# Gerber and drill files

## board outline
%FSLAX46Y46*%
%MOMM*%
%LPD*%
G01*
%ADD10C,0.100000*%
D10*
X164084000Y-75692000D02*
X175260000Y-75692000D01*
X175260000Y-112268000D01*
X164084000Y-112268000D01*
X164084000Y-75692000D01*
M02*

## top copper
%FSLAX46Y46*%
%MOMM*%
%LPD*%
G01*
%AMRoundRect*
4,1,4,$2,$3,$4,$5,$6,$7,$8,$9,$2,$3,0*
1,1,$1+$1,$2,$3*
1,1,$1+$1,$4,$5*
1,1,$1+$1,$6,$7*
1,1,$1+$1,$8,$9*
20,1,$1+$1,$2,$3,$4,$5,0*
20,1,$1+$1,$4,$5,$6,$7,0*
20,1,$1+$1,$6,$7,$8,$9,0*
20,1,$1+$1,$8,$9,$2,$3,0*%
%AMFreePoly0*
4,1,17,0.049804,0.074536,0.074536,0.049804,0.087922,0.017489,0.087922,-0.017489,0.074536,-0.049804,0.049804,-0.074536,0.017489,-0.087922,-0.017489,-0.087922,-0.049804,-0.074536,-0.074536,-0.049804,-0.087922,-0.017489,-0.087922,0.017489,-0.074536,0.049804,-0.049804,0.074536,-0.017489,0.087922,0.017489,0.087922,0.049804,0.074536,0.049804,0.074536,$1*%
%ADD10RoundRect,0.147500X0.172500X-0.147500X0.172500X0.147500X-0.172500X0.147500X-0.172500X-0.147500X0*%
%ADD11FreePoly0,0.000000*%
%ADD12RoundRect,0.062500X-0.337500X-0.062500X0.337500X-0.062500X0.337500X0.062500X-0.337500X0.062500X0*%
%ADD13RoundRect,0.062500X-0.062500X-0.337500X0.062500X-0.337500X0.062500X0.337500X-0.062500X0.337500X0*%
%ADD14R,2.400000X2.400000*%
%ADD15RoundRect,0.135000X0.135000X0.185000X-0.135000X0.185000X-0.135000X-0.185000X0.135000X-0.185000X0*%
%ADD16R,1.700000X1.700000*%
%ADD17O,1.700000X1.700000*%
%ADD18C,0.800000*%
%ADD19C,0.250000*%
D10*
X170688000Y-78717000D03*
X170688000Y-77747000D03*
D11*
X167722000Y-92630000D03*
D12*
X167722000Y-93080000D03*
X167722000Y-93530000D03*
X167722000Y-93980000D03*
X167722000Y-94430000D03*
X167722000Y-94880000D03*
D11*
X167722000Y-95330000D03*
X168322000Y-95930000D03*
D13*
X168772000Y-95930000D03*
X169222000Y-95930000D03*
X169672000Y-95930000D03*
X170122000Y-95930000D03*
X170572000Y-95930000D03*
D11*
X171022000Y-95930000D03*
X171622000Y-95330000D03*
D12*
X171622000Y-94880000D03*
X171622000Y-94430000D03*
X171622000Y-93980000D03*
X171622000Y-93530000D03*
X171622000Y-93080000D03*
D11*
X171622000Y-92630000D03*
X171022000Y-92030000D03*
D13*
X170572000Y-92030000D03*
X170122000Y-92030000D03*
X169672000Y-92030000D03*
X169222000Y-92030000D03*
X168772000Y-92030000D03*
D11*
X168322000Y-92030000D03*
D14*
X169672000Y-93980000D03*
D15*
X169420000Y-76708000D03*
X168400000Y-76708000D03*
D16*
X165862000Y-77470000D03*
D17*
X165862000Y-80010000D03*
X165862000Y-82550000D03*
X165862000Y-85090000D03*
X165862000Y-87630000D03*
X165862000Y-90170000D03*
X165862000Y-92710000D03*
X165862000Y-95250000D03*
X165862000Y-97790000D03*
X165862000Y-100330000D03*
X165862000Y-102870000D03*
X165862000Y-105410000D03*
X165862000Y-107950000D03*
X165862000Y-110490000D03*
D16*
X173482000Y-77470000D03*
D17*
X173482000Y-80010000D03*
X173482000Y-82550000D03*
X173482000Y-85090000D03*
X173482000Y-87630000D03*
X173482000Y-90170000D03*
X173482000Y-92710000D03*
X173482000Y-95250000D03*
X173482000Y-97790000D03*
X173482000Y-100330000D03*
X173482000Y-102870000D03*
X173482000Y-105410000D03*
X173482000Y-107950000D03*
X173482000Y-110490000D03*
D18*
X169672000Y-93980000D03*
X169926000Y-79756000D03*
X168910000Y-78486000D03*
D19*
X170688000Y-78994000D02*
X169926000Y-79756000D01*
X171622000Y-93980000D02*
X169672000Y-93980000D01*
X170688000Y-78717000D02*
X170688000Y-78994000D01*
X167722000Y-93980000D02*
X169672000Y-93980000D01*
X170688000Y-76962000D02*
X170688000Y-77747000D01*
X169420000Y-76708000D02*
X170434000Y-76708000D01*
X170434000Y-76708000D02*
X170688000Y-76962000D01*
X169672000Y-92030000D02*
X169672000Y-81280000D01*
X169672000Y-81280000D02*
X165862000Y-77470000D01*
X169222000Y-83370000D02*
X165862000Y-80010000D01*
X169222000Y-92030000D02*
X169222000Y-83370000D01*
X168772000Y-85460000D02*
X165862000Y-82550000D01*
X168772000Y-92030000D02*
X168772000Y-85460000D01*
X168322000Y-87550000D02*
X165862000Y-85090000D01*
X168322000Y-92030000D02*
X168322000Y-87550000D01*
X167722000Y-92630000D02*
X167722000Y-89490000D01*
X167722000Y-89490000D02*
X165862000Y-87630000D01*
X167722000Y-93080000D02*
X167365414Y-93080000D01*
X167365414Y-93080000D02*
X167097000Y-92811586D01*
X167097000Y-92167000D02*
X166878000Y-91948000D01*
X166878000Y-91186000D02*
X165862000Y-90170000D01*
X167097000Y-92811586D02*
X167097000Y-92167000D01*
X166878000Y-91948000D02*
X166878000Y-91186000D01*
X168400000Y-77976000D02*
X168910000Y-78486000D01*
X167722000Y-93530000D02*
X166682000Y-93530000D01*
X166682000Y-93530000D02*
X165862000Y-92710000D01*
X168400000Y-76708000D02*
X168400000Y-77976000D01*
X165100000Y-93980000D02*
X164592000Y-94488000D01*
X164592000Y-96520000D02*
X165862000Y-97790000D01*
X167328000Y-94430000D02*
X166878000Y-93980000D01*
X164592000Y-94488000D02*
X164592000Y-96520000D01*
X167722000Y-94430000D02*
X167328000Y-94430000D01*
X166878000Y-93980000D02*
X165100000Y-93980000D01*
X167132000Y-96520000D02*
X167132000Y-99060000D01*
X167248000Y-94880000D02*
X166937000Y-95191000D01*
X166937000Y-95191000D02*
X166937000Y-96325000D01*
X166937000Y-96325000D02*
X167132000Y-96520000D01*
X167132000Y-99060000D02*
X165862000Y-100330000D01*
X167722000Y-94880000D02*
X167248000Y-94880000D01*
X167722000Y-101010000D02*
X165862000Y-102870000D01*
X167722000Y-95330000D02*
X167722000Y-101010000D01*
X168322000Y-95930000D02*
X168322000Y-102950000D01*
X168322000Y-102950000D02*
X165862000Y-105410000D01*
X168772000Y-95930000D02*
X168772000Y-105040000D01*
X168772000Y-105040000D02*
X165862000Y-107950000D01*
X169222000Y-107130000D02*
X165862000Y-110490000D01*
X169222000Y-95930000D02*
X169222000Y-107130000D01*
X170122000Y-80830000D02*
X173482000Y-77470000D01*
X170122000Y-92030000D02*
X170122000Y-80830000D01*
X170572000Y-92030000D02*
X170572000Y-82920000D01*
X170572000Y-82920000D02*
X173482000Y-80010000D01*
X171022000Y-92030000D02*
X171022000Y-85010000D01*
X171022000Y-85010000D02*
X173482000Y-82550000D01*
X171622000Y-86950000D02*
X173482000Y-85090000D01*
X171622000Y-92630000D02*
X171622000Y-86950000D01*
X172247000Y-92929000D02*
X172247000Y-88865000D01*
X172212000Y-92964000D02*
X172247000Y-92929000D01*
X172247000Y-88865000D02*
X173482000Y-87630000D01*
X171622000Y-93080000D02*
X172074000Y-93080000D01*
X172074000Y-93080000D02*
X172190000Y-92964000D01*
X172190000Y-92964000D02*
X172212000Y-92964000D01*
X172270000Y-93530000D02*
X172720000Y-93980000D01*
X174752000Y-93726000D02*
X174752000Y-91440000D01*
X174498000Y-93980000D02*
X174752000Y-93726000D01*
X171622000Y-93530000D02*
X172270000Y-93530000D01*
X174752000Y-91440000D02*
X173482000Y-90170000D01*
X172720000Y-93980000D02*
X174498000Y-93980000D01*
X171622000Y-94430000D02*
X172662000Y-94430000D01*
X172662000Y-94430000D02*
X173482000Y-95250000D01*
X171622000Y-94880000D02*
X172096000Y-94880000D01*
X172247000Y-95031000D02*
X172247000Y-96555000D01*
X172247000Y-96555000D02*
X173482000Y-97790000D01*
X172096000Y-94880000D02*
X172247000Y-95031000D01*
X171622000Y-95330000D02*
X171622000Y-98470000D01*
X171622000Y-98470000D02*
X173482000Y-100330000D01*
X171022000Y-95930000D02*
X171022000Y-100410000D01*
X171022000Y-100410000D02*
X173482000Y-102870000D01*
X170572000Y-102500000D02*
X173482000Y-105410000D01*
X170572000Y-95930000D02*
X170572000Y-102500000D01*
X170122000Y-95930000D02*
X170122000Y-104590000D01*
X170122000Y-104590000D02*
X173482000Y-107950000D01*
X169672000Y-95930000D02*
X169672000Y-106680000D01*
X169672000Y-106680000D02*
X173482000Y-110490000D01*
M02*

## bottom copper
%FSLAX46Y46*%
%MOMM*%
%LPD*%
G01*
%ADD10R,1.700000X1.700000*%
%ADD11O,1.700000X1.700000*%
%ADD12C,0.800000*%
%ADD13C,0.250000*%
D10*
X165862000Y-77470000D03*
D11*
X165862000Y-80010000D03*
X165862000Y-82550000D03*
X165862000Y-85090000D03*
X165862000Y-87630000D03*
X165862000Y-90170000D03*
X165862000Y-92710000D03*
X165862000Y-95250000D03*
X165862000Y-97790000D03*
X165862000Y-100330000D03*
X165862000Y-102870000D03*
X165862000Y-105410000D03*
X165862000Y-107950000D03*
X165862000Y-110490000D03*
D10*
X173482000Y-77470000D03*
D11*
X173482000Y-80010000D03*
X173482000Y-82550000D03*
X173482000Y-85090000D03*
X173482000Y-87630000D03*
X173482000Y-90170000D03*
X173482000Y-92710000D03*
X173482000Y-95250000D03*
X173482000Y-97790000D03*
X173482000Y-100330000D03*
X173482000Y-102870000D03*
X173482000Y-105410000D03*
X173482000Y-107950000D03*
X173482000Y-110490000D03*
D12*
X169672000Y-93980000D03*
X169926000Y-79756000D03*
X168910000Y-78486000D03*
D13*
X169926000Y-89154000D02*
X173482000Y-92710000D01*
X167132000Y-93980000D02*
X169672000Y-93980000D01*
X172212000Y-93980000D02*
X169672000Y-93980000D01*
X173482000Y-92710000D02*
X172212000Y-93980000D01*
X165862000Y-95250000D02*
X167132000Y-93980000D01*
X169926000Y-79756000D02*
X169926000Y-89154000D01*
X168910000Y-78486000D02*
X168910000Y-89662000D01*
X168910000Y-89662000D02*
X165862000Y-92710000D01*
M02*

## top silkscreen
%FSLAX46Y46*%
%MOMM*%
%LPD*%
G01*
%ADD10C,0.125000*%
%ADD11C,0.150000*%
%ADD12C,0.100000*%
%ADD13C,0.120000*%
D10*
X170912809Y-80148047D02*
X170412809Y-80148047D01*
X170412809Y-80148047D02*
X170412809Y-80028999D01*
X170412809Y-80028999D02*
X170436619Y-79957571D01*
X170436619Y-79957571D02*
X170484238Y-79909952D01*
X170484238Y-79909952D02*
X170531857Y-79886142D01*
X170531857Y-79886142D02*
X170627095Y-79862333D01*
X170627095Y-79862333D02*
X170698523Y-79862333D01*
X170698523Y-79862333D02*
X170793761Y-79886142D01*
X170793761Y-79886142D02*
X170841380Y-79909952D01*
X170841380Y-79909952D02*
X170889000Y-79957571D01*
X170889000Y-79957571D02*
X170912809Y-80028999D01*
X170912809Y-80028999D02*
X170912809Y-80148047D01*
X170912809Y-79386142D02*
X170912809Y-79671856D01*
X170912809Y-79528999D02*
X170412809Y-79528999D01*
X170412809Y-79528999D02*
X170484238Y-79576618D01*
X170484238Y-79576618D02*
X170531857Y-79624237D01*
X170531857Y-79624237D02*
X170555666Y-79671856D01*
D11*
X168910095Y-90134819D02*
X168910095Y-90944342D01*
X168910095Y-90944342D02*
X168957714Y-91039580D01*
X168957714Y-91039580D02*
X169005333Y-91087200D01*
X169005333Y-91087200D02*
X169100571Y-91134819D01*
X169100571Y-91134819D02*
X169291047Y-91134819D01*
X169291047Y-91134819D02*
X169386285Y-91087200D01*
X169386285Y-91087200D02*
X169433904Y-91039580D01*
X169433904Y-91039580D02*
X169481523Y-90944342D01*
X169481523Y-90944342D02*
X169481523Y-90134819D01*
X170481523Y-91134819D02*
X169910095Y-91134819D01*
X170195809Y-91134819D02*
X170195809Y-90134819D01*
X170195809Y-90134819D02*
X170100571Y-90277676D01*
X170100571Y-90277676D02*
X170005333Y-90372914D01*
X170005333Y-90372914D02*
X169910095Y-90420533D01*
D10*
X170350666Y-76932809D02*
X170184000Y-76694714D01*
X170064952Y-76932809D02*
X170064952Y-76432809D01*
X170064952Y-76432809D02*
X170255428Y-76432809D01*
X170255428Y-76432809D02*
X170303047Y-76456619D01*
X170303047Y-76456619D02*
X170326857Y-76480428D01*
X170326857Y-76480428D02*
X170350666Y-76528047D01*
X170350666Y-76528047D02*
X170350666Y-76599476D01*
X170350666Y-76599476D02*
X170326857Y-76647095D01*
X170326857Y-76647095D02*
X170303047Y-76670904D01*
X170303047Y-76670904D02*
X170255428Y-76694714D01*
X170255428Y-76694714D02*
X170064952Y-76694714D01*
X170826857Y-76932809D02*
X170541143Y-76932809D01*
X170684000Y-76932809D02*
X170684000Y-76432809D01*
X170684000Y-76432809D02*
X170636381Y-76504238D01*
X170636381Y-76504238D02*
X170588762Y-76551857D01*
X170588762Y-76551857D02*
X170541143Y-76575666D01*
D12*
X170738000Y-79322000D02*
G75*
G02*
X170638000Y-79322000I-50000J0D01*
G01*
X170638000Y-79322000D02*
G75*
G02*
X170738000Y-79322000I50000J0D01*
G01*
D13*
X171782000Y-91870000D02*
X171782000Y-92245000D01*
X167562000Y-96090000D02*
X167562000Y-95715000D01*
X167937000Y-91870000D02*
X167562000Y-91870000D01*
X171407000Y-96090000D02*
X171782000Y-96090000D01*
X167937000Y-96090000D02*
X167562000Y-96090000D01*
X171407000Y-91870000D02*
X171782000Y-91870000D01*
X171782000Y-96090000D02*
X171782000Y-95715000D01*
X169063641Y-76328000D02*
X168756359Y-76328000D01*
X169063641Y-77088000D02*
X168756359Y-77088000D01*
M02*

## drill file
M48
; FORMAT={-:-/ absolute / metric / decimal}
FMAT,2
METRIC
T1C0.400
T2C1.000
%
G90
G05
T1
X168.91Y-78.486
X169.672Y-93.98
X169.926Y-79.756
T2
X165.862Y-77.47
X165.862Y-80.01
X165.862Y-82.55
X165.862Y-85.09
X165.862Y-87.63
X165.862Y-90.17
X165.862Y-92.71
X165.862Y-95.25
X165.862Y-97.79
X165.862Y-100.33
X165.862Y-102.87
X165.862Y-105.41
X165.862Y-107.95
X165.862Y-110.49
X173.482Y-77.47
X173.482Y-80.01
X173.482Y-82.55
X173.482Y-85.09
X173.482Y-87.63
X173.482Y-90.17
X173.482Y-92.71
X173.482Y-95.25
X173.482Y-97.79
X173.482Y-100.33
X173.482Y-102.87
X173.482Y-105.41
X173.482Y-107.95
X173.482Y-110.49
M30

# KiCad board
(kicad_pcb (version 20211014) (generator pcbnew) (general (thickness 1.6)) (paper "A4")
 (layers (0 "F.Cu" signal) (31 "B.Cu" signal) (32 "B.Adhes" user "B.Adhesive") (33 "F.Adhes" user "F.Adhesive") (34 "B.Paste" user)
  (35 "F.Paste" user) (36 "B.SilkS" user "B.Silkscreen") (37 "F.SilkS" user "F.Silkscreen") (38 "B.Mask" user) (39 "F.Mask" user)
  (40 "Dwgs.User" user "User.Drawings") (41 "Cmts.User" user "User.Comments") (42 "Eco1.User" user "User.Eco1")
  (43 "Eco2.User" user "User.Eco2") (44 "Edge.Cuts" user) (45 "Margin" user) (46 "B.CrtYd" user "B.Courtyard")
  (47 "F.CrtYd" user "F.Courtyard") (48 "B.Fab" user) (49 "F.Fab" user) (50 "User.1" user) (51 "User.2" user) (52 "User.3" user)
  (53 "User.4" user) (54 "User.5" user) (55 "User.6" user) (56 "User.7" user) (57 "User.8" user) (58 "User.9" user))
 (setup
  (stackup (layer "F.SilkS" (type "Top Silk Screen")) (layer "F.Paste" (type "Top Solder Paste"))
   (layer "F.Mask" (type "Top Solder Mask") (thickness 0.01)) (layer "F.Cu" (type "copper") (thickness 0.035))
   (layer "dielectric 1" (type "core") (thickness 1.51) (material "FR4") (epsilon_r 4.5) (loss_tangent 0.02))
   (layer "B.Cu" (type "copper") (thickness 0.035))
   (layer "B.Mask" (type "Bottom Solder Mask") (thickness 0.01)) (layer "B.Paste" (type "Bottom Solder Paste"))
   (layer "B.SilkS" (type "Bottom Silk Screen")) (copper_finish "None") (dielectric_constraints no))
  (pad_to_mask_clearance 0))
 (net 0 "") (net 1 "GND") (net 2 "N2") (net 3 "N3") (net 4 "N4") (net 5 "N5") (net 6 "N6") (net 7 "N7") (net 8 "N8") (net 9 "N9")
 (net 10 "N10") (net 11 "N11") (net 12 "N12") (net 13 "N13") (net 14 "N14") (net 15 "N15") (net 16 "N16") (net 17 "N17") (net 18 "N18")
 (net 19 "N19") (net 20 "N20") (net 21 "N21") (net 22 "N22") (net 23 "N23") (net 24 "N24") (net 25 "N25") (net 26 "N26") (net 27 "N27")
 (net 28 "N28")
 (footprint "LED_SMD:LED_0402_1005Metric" (layer "F.Cu") (at 170.688 78.232 90)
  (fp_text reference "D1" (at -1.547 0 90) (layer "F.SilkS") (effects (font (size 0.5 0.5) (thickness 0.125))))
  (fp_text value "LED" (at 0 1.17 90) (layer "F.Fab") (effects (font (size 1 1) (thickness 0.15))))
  (fp_circle (center -1.09 0) (end -1.04 0) (layer "F.SilkS") (width 0.1) (fill none))
  (pad "1" smd roundrect (at -0.485 0 90) (size 0.59 0.64) (layers "F.Cu" "F.Paste" "F.Mask") (roundrect_rratio 0.25) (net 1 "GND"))
  (pad "2" smd roundrect (at 0.485 0 90) (size 0.59 0.64) (layers "F.Cu" "F.Paste" "F.Mask") (roundrect_rratio 0.25) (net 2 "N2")))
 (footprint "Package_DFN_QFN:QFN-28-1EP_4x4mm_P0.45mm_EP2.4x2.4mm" (layer "F.Cu") (at 169.672 93.98)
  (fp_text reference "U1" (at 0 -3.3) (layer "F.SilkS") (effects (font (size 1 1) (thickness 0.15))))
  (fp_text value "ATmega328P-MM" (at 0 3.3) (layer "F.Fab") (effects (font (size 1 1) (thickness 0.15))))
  (fp_line (start 2.11 -2.11) (end 2.11 -1.735) (layer "F.SilkS") (width 0.12))
  (fp_line (start -2.11 2.11) (end -2.11 1.735) (layer "F.SilkS") (width 0.12))
  (fp_line (start -1.735 -2.11) (end -2.11 -2.11) (layer "F.SilkS") (width 0.12))
  (fp_line (start 1.735 2.11) (end 2.11 2.11) (layer "F.SilkS") (width 0.12))
  (fp_line (start -1.735 2.11) (end -2.11 2.11) (layer "F.SilkS") (width 0.12))
  (fp_line (start 1.735 -2.11) (end 2.11 -2.11) (layer "F.SilkS") (width 0.12))
  (fp_line (start 2.11 2.11) (end 2.11 1.735) (layer "F.SilkS") (width 0.12))
  (pad "" smd roundrect (at -0.6 -0.6) (size 0.97 0.97) (layers "F.Paste") (roundrect_rratio 0.25))
  (pad "" smd roundrect (at 0.6 0.6) (size 0.97 0.97) (layers "F.Paste") (roundrect_rratio 0.25))
  (pad "" smd roundrect (at 0.6 -0.6) (size 0.97 0.97) (layers "F.Paste") (roundrect_rratio 0.25))
  (pad "" smd roundrect (at -0.6 0.6) (size 0.97 0.97) (layers "F.Paste") (roundrect_rratio 0.25))
  (pad "1" smd custom (at -1.95 -1.35) (size 0.179289 0.179289) (layers "F.Cu" "F.Paste" "F.Mask") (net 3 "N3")
   (options (clearance outline) (anchor circle)) (primitives))
  (pad "2" smd roundrect (at -1.95 -0.9) (size 0.8 0.25) (layers "F.Cu" "F.Paste" "F.Mask") (roundrect_rratio 0.25) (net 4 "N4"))
  (pad "3" smd roundrect (at -1.95 -0.45) (size 0.8 0.25) (layers "F.Cu" "F.Paste" "F.Mask") (roundrect_rratio 0.25) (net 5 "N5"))
  (pad "4" smd roundrect (at -1.95 0) (size 0.8 0.25) (layers "F.Cu" "F.Paste" "F.Mask") (roundrect_rratio 0.25) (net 1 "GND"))
  (pad "5" smd roundrect (at -1.95 0.45) (size 0.8 0.25) (layers "F.Cu" "F.Paste" "F.Mask") (roundrect_rratio 0.25) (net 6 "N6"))
  (pad "6" smd roundrect (at -1.95 0.9) (size 0.8 0.25) (layers "F.Cu" "F.Paste" "F.Mask") (roundrect_rratio 0.25) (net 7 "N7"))
  (pad "7" smd custom (at -1.95 1.35) (size 0.179289 0.179289) (layers "F.Cu" "F.Paste" "F.Mask") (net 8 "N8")
   (options (clearance outline) (anchor circle)) (primitives))
  (pad "8" smd custom (at -1.35 1.95) (size 0.179289 0.179289) (layers "F.Cu" "F.Paste" "F.Mask") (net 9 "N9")
   (options (clearance outline) (anchor circle)) (primitives))
  (pad "9" smd roundrect (at -0.9 1.95) (size 0.25 0.8) (layers "F.Cu" "F.Paste" "F.Mask") (roundrect_rratio 0.25) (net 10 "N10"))
  (pad "10" smd roundrect (at -0.45 1.95) (size 0.25 0.8) (layers "F.Cu" "F.Paste" "F.Mask") (roundrect_rratio 0.25) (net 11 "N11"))
  (pad "11" smd roundrect (at 0 1.95) (size 0.25 0.8) (layers "F.Cu" "F.Paste" "F.Mask") (roundrect_rratio 0.25) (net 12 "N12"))
  (pad "12" smd roundrect (at 0.45 1.95) (size 0.25 0.8) (layers "F.Cu" "F.Paste" "F.Mask") (roundrect_rratio 0.25) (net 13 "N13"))
  (pad "13" smd roundrect (at 0.9 1.95) (size 0.25 0.8) (layers "F.Cu" "F.Paste" "F.Mask") (roundrect_rratio 0.25) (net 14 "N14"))
  (pad "14" smd custom (at 1.35 1.95) (size 0.179289 0.179289) (layers "F.Cu" "F.Paste" "F.Mask") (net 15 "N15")
   (options (clearance outline) (anchor circle)) (primitives))
  (pad "15" smd custom (at 1.95 1.35) (size 0.179289 0.179289) (layers "F.Cu" "F.Paste" "F.Mask") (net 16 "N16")
   (options (clearance outline) (anchor circle)) (primitives))
  (pad "16" smd roundrect (at 1.95 0.9) (size 0.8 0.25) (layers "F.Cu" "F.Paste" "F.Mask") (roundrect_rratio 0.25) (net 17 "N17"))
  (pad "17" smd roundrect (at 1.95 0.45) (size 0.8 0.25) (layers "F.Cu" "F.Paste" "F.Mask") (roundrect_rratio 0.25) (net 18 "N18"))
  (pad "18" smd roundrect (at 1.95 0) (size 0.8 0.25) (layers "F.Cu" "F.Paste" "F.Mask") (roundrect_rratio 0.25) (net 1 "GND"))
  (pad "19" smd roundrect (at 1.95 -0.45) (size 0.8 0.25) (layers "F.Cu" "F.Paste" "F.Mask") (roundrect_rratio 0.25) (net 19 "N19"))
  (pad "20" smd roundrect (at 1.95 -0.9) (size 0.8 0.25) (layers "F.Cu" "F.Paste" "F.Mask") (roundrect_rratio 0.25) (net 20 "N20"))
  (pad "21" smd custom (at 1.95 -1.35) (size 0.179289 0.179289) (layers "F.Cu" "F.Paste" "F.Mask") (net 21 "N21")
   (options (clearance outline) (anchor circle)) (primitives))
  (pad "22" smd custom (at 1.35 -1.95) (size 0.179289 0.179289) (layers "F.Cu" "F.Paste" "F.Mask") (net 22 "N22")
   (options (clearance outline) (anchor circle)) (primitives))
  (pad "23" smd roundrect (at 0.9 -1.95) (size 0.25 0.8) (layers "F.Cu" "F.Paste" "F.Mask") (roundrect_rratio 0.25) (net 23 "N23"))
  (pad "24" smd roundrect (at 0.45 -1.95) (size 0.25 0.8) (layers "F.Cu" "F.Paste" "F.Mask") (roundrect_rratio 0.25) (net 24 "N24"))
  (pad "25" smd roundrect (at 0 -1.95) (size 0.25 0.8) (layers "F.Cu" "F.Paste" "F.Mask") (roundrect_rratio 0.25) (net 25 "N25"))
  (pad "26" smd roundrect (at -0.45 -1.95) (size 0.25 0.8) (layers "F.Cu" "F.Paste" "F.Mask") (roundrect_rratio 0.25) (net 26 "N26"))
  (pad "27" smd roundrect (at -0.9 -1.95) (size 0.25 0.8) (layers "F.Cu" "F.Paste" "F.Mask") (roundrect_rratio 0.25) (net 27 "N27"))
  (pad "28" smd custom (at -1.35 -1.95) (size 0.179289 0.179289) (layers "F.Cu" "F.Paste" "F.Mask") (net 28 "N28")
   (options (clearance outline) (anchor circle)) (primitives))
  (pad "29" smd rect (at 0 0) (size 2.4 2.4) (layers "F.Cu" "F.Mask") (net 1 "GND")))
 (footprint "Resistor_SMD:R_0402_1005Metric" (layer "F.Cu") (at 168.91 76.708 180)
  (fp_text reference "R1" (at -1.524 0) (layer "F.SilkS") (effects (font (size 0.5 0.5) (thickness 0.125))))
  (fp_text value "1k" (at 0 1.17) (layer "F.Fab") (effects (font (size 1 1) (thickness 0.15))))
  (fp_line (start -0.153641 0.38) (end 0.153641 0.38) (layer "F.SilkS") (width 0.12))
  (fp_line (start -0.153641 -0.38) (end 0.153641 -0.38) (layer "F.SilkS") (width 0.12))
  (pad "1" smd roundrect (at -0.51 0 180) (size 0.54 0.64) (layers "F.Cu" "F.Paste" "F.Mask") (roundrect_rratio 0.25) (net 2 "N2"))
  (pad "2" smd roundrect (at 0.51 0 180) (size 0.54 0.64) (layers "F.Cu" "F.Paste" "F.Mask") (roundrect_rratio 0.25) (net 5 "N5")))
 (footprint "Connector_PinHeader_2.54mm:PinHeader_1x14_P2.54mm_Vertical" (layer "B.Cu") (at 165.862 77.47 180)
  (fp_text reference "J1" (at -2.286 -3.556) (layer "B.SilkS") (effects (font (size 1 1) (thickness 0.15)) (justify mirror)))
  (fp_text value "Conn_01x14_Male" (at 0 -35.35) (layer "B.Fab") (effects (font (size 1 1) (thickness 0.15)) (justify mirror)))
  (pad "1" thru_hole rect (at 0 0 180) (size 1.7 1.7) (drill 1) (layers *.Cu *.Mask) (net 25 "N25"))
  (pad "2" thru_hole oval (at 0 -2.54 180) (size 1.7 1.7) (drill 1) (layers *.Cu *.Mask) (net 26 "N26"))
  (pad "3" thru_hole oval (at 0 -5.08 180) (size 1.7 1.7) (drill 1) (layers *.Cu *.Mask) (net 27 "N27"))
  (pad "4" thru_hole oval (at 0 -7.62 180) (size 1.7 1.7) (drill 1) (layers *.Cu *.Mask) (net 28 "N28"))
  (pad "5" thru_hole oval (at 0 -10.16 180) (size 1.7 1.7) (drill 1) (layers *.Cu *.Mask) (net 3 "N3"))
  (pad "6" thru_hole oval (at 0 -12.7 180) (size 1.7 1.7) (drill 1) (layers *.Cu *.Mask) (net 4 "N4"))
  (pad "7" thru_hole oval (at 0 -15.24 180) (size 1.7 1.7) (drill 1) (layers *.Cu *.Mask) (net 5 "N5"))
  (pad "8" thru_hole oval (at 0 -17.78 180) (size 1.7 1.7) (drill 1) (layers *.Cu *.Mask) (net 1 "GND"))
  (pad "9" thru_hole oval (at 0 -20.32 180) (size 1.7 1.7) (drill 1) (layers *.Cu *.Mask) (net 6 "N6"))
  (pad "10" thru_hole oval (at 0 -22.86 180) (size 1.7 1.7) (drill 1) (layers *.Cu *.Mask) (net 7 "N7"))
  (pad "11" thru_hole oval (at 0 -25.4 180) (size 1.7 1.7) (drill 1) (layers *.Cu *.Mask) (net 8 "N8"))
  (pad "12" thru_hole oval (at 0 -27.94 180) (size 1.7 1.7) (drill 1) (layers *.Cu *.Mask) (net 9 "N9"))
  (pad "13" thru_hole oval (at 0 -30.48 180) (size 1.7 1.7) (drill 1) (layers *.Cu *.Mask) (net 10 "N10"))
  (pad "14" thru_hole oval (at 0 -33.02 180) (size 1.7 1.7) (drill 1) (layers *.Cu *.Mask) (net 11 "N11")))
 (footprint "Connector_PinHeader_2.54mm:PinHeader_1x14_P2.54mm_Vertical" (layer "B.Cu") (at 173.482 77.47 180)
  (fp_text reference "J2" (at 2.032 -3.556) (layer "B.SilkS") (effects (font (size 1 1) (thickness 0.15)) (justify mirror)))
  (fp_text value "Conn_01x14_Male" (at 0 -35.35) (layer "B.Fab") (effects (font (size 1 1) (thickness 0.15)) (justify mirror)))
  (pad "1" thru_hole rect (at 0 0 180) (size 1.7 1.7) (drill 1) (layers *.Cu *.Mask) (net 24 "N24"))
  (pad "2" thru_hole oval (at 0 -2.54 180) (size 1.7 1.7) (drill 1) (layers *.Cu *.Mask) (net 23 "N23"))
  (pad "3" thru_hole oval (at 0 -5.08 180) (size 1.7 1.7) (drill 1) (layers *.Cu *.Mask) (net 22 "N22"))
  (pad "4" thru_hole oval (at 0 -7.62 180) (size 1.7 1.7) (drill 1) (layers *.Cu *.Mask) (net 21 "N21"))
  (pad "5" thru_hole oval (at 0 -10.16 180) (size 1.7 1.7) (drill 1) (layers *.Cu *.Mask) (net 20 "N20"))
  (pad "6" thru_hole oval (at 0 -12.7 180) (size 1.7 1.7) (drill 1) (layers *.Cu *.Mask) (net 19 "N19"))
  (pad "7" thru_hole oval (at 0 -15.24 180) (size 1.7 1.7) (drill 1) (layers *.Cu *.Mask) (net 1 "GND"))
  (pad "8" thru_hole oval (at 0 -17.78 180) (size 1.7 1.7) (drill 1) (layers *.Cu *.Mask) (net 18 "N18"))
  (pad "9" thru_hole oval (at 0 -20.32 180) (size 1.7 1.7) (drill 1) (layers *.Cu *.Mask) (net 17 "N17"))
  (pad "10" thru_hole oval (at 0 -22.86 180) (size 1.7 1.7) (drill 1) (layers *.Cu *.Mask) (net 16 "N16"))
  (pad "11" thru_hole oval (at 0 -25.4 180) (size 1.7 1.7) (drill 1) (layers *.Cu *.Mask) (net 15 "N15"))
  (pad "12" thru_hole oval (at 0 -27.94 180) (size 1.7 1.7) (drill 1) (layers *.Cu *.Mask) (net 14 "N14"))
  (pad "13" thru_hole oval (at 0 -30.48 180) (size 1.7 1.7) (drill 1) (layers *.Cu *.Mask) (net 13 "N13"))
  (pad "14" thru_hole oval (at 0 -33.02 180) (size 1.7 1.7) (drill 1) (layers *.Cu *.Mask) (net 12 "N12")))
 (gr_rect (start 164.084 75.692) (end 175.26 112.268) (layer "Edge.Cuts") (width 0.1) (fill none))
 (segment (start 170.688 78.994) (end 169.926 79.756) (width 0.25) (layer "F.Cu") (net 1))
 (segment (start 171.622 93.98) (end 169.672 93.98) (width 0.25) (layer "F.Cu") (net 1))
 (segment (start 170.688 78.717) (end 170.688 78.994) (width 0.25) (layer "F.Cu") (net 1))
 (segment (start 167.722 93.98) (end 169.672 93.98) (width 0.25) (layer "F.Cu") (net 1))
 (via (at 169.672 93.98) (size 0.8) (drill 0.4) (layers "F.Cu" "B.Cu") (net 1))
 (via (at 169.926 79.756) (size 0.8) (drill 0.4) (layers "F.Cu" "B.Cu") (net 1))
 (segment (start 169.926 89.154) (end 173.482 92.71) (width 0.25) (layer "B.Cu") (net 1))
 (segment (start 167.132 93.98) (end 169.672 93.98) (width 0.25) (layer "B.Cu") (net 1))
 (segment (start 172.212 93.98) (end 169.672 93.98) (width 0.25) (layer "B.Cu") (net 1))
 (segment (start 173.482 92.71) (end 172.212 93.98) (width 0.25) (layer "B.Cu") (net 1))
 (segment (start 165.862 95.25) (end 167.132 93.98) (width 0.25) (layer "B.Cu") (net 1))
 (segment (start 169.926 79.756) (end 169.926 89.154) (width 0.25) (layer "B.Cu") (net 1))
 (segment (start 170.688 76.962) (end 170.688 77.747) (width 0.25) (layer "F.Cu") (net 2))
 (segment (start 169.42 76.708) (end 170.434 76.708) (width 0.25) (layer "F.Cu") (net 2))
 (segment (start 170.434 76.708) (end 170.688 76.962) (width 0.25) (layer "F.Cu") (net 2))
 (segment (start 169.672 92.03) (end 169.672 81.28) (width 0.25) (layer "F.Cu") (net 25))
 (segment (start 169.672 81.28) (end 165.862 77.47) (width 0.25) (layer "F.Cu") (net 25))
 (segment (start 169.222 83.37) (end 165.862 80.01) (width 0.25) (layer "F.Cu") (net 26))
 (segment (start 169.222 92.03) (end 169.222 83.37) (width 0.25) (layer "F.Cu") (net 26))
 (segment (start 168.772 85.46) (end 165.862 82.55) (width 0.25) (layer "F.Cu") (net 27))
 (segment (start 168.772 92.03) (end 168.772 85.46) (width 0.25) (layer "F.Cu") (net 27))
 (segment (start 168.322 87.55) (end 165.862 85.09) (width 0.25) (layer "F.Cu") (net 28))
 (segment (start 168.322 92.03) (end 168.322 87.55) (width 0.25) (layer "F.Cu") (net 28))
 (segment (start 167.722 92.63) (end 167.722 89.49) (width 0.25) (layer "F.Cu") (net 3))
 (segment (start 167.722 89.49) (end 165.862 87.63) (width 0.25) (layer "F.Cu") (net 3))
 (segment (start 167.722 93.08) (end 167.365414 93.08) (width 0.25) (layer "F.Cu") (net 4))
 (segment (start 167.365414 93.08) (end 167.097 92.811586) (width 0.25) (layer "F.Cu") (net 4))
 (segment (start 167.097 92.167) (end 166.878 91.948) (width 0.25) (layer "F.Cu") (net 4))
 (segment (start 166.878 91.186) (end 165.862 90.17) (width 0.25) (layer "F.Cu") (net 4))
 (segment (start 167.097 92.811586) (end 167.097 92.167) (width 0.25) (layer "F.Cu") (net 4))
 (segment (start 166.878 91.948) (end 166.878 91.186) (width 0.25) (layer "F.Cu") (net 4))
 (segment (start 168.4 77.976) (end 168.91 78.486) (width 0.25) (layer "F.Cu") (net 5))
 (segment (start 167.722 93.53) (end 166.682 93.53) (width 0.25) (layer "F.Cu") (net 5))
 (segment (start 166.682 93.53) (end 165.862 92.71) (width 0.25) (layer "F.Cu") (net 5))
 (segment (start 168.4 76.708) (end 168.4 77.976) (width 0.25) (layer "F.Cu") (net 5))
 (via (at 168.91 78.486) (size 0.8) (drill 0.4) (layers "F.Cu" "B.Cu") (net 5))
 (segment (start 168.91 78.486) (end 168.91 89.662) (width 0.25) (layer "B.Cu") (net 5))
 (segment (start 168.91 89.662) (end 165.862 92.71) (width 0.25) (layer "B.Cu") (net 5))
 (segment (start 165.1 93.98) (end 164.592 94.488) (width 0.25) (layer "F.Cu") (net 6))
 (segment (start 164.592 96.52) (end 165.862 97.79) (width 0.25) (layer "F.Cu") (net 6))
 (segment (start 167.328 94.43) (end 166.878 93.98) (width 0.25) (layer "F.Cu") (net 6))
 (segment (start 164.592 94.488) (end 164.592 96.52) (width 0.25) (layer "F.Cu") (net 6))
 (segment (start 167.722 94.43) (end 167.328 94.43) (width 0.25) (layer "F.Cu") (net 6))
 (segment (start 166.878 93.98) (end 165.1 93.98) (width 0.25) (layer "F.Cu") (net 6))
 (segment (start 167.132 96.52) (end 167.132 99.06) (width 0.25) (layer "F.Cu") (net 7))
 (segment (start 167.248 94.88) (end 166.937 95.191) (width 0.25) (layer "F.Cu") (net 7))
 (segment (start 166.937 95.191) (end 166.937 96.325) (width 0.25) (layer "F.Cu") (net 7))
 (segment (start 166.937 96.325) (end 167.132 96.52) (width 0.25) (layer "F.Cu") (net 7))
 (segment (start 167.132 99.06) (end 165.862 100.33) (width 0.25) (layer "F.Cu") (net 7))
 (segment (start 167.722 94.88) (end 167.248 94.88) (width 0.25) (layer "F.Cu") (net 7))
 (segment (start 167.722 101.01) (end 165.862 102.87) (width 0.25) (layer "F.Cu") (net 8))
 (segment (start 167.722 95.33) (end 167.722 101.01) (width 0.25) (layer "F.Cu") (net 8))
 (segment (start 168.322 95.93) (end 168.322 102.95) (width 0.25) (layer "F.Cu") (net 9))
 (segment (start 168.322 102.95) (end 165.862 105.41) (width 0.25) (layer "F.Cu") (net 9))
 (segment (start 168.772 95.93) (end 168.772 105.04) (width 0.25) (layer "F.Cu") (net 10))
 (segment (start 168.772 105.04) (end 165.862 107.95) (width 0.25) (layer "F.Cu") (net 10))
 (segment (start 169.222 107.13) (end 165.862 110.49) (width 0.25) (layer "F.Cu") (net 11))
 (segment (start 169.222 95.93) (end 169.222 107.13) (width 0.25) (layer "F.Cu") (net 11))
 (segment (start 170.122 80.83) (end 173.482 77.47) (width 0.25) (layer "F.Cu") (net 24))
 (segment (start 170.122 92.03) (end 170.122 80.83) (width 0.25) (layer "F.Cu") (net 24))
 (segment (start 170.572 92.03) (end 170.572 82.92) (width 0.25) (layer "F.Cu") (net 23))
 (segment (start 170.572 82.92) (end 173.482 80.01) (width 0.25) (layer "F.Cu") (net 23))
 (segment (start 171.022 92.03) (end 171.022 85.01) (width 0.25) (layer "F.Cu") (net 22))
 (segment (start 171.022 85.01) (end 173.482 82.55) (width 0.25) (layer "F.Cu") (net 22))
 (segment (start 171.622 86.95) (end 173.482 85.09) (width 0.25) (layer "F.Cu") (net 21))
 (segment (start 171.622 92.63) (end 171.622 86.95) (width 0.25) (layer "F.Cu") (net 21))
 (segment (start 172.247 92.929) (end 172.247 88.865) (width 0.25) (layer "F.Cu") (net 20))
 (segment (start 172.212 92.964) (end 172.247 92.929) (width 0.25) (layer "F.Cu") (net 20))
 (segment (start 172.247 88.865) (end 173.482 87.63) (width 0.25) (layer "F.Cu") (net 20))
 (segment (start 171.622 93.08) (end 172.074 93.08) (width 0.25) (layer "F.Cu") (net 20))
 (segment (start 172.074 93.08) (end 172.19 92.964) (width 0.25) (layer "F.Cu") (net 20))
 (segment (start 172.19 92.964) (end 172.212 92.964) (width 0.25) (layer "F.Cu") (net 20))
 (segment (start 172.27 93.53) (end 172.72 93.98) (width 0.25) (layer "F.Cu") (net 19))
 (segment (start 174.752 93.726) (end 174.752 91.44) (width 0.25) (layer "F.Cu") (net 19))
 (segment (start 174.498 93.98) (end 174.752 93.726) (width 0.25) (layer "F.Cu") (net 19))
 (segment (start 171.622 93.53) (end 172.27 93.53) (width 0.25) (layer "F.Cu") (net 19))
 (segment (start 174.752 91.44) (end 173.482 90.17) (width 0.25) (layer "F.Cu") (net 19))
 (segment (start 172.72 93.98) (end 174.498 93.98) (width 0.25) (layer "F.Cu") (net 19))
 (segment (start 171.622 94.43) (end 172.662 94.43) (width 0.25) (layer "F.Cu") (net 18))
 (segment (start 172.662 94.43) (end 173.482 95.25) (width 0.25) (layer "F.Cu") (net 18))
 (segment (start 171.622 94.88) (end 172.096 94.88) (width 0.25) (layer "F.Cu") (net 17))
 (segment (start 172.247 95.031) (end 172.247 96.555) (width 0.25) (layer "F.Cu") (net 17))
 (segment (start 172.247 96.555) (end 173.482 97.79) (width 0.25) (layer "F.Cu") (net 17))
 (segment (start 172.096 94.88) (end 172.247 95.031) (width 0.25) (layer "F.Cu") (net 17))
 (segment (start 171.622 95.33) (end 171.622 98.47) (width 0.25) (layer "F.Cu") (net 16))
 (segment (start 171.622 98.47) (end 173.482 100.33) (width 0.25) (layer "F.Cu") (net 16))
 (segment (start 171.022 95.93) (end 171.022 100.41) (width 0.25) (layer "F.Cu") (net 15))
 (segment (start 171.022 100.41) (end 173.482 102.87) (width 0.25) (layer "F.Cu") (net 15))
 (segment (start 170.572 102.5) (end 173.482 105.41) (width 0.25) (layer "F.Cu") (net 14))
 (segment (start 170.572 95.93) (end 170.572 102.5) (width 0.25) (layer "F.Cu") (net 14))
 (segment (start 170.122 95.93) (end 170.122 104.59) (width 0.25) (layer "F.Cu") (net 13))
 (segment (start 170.122 104.59) (end 173.482 107.95) (width 0.25) (layer "F.Cu") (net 13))
 (segment (start 169.672 95.93) (end 169.672 106.68) (width 0.25) (layer "F.Cu") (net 12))
 (segment (start 169.672 106.68) (end 173.482 110.49) (width 0.25) (layer "F.Cu") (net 12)))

